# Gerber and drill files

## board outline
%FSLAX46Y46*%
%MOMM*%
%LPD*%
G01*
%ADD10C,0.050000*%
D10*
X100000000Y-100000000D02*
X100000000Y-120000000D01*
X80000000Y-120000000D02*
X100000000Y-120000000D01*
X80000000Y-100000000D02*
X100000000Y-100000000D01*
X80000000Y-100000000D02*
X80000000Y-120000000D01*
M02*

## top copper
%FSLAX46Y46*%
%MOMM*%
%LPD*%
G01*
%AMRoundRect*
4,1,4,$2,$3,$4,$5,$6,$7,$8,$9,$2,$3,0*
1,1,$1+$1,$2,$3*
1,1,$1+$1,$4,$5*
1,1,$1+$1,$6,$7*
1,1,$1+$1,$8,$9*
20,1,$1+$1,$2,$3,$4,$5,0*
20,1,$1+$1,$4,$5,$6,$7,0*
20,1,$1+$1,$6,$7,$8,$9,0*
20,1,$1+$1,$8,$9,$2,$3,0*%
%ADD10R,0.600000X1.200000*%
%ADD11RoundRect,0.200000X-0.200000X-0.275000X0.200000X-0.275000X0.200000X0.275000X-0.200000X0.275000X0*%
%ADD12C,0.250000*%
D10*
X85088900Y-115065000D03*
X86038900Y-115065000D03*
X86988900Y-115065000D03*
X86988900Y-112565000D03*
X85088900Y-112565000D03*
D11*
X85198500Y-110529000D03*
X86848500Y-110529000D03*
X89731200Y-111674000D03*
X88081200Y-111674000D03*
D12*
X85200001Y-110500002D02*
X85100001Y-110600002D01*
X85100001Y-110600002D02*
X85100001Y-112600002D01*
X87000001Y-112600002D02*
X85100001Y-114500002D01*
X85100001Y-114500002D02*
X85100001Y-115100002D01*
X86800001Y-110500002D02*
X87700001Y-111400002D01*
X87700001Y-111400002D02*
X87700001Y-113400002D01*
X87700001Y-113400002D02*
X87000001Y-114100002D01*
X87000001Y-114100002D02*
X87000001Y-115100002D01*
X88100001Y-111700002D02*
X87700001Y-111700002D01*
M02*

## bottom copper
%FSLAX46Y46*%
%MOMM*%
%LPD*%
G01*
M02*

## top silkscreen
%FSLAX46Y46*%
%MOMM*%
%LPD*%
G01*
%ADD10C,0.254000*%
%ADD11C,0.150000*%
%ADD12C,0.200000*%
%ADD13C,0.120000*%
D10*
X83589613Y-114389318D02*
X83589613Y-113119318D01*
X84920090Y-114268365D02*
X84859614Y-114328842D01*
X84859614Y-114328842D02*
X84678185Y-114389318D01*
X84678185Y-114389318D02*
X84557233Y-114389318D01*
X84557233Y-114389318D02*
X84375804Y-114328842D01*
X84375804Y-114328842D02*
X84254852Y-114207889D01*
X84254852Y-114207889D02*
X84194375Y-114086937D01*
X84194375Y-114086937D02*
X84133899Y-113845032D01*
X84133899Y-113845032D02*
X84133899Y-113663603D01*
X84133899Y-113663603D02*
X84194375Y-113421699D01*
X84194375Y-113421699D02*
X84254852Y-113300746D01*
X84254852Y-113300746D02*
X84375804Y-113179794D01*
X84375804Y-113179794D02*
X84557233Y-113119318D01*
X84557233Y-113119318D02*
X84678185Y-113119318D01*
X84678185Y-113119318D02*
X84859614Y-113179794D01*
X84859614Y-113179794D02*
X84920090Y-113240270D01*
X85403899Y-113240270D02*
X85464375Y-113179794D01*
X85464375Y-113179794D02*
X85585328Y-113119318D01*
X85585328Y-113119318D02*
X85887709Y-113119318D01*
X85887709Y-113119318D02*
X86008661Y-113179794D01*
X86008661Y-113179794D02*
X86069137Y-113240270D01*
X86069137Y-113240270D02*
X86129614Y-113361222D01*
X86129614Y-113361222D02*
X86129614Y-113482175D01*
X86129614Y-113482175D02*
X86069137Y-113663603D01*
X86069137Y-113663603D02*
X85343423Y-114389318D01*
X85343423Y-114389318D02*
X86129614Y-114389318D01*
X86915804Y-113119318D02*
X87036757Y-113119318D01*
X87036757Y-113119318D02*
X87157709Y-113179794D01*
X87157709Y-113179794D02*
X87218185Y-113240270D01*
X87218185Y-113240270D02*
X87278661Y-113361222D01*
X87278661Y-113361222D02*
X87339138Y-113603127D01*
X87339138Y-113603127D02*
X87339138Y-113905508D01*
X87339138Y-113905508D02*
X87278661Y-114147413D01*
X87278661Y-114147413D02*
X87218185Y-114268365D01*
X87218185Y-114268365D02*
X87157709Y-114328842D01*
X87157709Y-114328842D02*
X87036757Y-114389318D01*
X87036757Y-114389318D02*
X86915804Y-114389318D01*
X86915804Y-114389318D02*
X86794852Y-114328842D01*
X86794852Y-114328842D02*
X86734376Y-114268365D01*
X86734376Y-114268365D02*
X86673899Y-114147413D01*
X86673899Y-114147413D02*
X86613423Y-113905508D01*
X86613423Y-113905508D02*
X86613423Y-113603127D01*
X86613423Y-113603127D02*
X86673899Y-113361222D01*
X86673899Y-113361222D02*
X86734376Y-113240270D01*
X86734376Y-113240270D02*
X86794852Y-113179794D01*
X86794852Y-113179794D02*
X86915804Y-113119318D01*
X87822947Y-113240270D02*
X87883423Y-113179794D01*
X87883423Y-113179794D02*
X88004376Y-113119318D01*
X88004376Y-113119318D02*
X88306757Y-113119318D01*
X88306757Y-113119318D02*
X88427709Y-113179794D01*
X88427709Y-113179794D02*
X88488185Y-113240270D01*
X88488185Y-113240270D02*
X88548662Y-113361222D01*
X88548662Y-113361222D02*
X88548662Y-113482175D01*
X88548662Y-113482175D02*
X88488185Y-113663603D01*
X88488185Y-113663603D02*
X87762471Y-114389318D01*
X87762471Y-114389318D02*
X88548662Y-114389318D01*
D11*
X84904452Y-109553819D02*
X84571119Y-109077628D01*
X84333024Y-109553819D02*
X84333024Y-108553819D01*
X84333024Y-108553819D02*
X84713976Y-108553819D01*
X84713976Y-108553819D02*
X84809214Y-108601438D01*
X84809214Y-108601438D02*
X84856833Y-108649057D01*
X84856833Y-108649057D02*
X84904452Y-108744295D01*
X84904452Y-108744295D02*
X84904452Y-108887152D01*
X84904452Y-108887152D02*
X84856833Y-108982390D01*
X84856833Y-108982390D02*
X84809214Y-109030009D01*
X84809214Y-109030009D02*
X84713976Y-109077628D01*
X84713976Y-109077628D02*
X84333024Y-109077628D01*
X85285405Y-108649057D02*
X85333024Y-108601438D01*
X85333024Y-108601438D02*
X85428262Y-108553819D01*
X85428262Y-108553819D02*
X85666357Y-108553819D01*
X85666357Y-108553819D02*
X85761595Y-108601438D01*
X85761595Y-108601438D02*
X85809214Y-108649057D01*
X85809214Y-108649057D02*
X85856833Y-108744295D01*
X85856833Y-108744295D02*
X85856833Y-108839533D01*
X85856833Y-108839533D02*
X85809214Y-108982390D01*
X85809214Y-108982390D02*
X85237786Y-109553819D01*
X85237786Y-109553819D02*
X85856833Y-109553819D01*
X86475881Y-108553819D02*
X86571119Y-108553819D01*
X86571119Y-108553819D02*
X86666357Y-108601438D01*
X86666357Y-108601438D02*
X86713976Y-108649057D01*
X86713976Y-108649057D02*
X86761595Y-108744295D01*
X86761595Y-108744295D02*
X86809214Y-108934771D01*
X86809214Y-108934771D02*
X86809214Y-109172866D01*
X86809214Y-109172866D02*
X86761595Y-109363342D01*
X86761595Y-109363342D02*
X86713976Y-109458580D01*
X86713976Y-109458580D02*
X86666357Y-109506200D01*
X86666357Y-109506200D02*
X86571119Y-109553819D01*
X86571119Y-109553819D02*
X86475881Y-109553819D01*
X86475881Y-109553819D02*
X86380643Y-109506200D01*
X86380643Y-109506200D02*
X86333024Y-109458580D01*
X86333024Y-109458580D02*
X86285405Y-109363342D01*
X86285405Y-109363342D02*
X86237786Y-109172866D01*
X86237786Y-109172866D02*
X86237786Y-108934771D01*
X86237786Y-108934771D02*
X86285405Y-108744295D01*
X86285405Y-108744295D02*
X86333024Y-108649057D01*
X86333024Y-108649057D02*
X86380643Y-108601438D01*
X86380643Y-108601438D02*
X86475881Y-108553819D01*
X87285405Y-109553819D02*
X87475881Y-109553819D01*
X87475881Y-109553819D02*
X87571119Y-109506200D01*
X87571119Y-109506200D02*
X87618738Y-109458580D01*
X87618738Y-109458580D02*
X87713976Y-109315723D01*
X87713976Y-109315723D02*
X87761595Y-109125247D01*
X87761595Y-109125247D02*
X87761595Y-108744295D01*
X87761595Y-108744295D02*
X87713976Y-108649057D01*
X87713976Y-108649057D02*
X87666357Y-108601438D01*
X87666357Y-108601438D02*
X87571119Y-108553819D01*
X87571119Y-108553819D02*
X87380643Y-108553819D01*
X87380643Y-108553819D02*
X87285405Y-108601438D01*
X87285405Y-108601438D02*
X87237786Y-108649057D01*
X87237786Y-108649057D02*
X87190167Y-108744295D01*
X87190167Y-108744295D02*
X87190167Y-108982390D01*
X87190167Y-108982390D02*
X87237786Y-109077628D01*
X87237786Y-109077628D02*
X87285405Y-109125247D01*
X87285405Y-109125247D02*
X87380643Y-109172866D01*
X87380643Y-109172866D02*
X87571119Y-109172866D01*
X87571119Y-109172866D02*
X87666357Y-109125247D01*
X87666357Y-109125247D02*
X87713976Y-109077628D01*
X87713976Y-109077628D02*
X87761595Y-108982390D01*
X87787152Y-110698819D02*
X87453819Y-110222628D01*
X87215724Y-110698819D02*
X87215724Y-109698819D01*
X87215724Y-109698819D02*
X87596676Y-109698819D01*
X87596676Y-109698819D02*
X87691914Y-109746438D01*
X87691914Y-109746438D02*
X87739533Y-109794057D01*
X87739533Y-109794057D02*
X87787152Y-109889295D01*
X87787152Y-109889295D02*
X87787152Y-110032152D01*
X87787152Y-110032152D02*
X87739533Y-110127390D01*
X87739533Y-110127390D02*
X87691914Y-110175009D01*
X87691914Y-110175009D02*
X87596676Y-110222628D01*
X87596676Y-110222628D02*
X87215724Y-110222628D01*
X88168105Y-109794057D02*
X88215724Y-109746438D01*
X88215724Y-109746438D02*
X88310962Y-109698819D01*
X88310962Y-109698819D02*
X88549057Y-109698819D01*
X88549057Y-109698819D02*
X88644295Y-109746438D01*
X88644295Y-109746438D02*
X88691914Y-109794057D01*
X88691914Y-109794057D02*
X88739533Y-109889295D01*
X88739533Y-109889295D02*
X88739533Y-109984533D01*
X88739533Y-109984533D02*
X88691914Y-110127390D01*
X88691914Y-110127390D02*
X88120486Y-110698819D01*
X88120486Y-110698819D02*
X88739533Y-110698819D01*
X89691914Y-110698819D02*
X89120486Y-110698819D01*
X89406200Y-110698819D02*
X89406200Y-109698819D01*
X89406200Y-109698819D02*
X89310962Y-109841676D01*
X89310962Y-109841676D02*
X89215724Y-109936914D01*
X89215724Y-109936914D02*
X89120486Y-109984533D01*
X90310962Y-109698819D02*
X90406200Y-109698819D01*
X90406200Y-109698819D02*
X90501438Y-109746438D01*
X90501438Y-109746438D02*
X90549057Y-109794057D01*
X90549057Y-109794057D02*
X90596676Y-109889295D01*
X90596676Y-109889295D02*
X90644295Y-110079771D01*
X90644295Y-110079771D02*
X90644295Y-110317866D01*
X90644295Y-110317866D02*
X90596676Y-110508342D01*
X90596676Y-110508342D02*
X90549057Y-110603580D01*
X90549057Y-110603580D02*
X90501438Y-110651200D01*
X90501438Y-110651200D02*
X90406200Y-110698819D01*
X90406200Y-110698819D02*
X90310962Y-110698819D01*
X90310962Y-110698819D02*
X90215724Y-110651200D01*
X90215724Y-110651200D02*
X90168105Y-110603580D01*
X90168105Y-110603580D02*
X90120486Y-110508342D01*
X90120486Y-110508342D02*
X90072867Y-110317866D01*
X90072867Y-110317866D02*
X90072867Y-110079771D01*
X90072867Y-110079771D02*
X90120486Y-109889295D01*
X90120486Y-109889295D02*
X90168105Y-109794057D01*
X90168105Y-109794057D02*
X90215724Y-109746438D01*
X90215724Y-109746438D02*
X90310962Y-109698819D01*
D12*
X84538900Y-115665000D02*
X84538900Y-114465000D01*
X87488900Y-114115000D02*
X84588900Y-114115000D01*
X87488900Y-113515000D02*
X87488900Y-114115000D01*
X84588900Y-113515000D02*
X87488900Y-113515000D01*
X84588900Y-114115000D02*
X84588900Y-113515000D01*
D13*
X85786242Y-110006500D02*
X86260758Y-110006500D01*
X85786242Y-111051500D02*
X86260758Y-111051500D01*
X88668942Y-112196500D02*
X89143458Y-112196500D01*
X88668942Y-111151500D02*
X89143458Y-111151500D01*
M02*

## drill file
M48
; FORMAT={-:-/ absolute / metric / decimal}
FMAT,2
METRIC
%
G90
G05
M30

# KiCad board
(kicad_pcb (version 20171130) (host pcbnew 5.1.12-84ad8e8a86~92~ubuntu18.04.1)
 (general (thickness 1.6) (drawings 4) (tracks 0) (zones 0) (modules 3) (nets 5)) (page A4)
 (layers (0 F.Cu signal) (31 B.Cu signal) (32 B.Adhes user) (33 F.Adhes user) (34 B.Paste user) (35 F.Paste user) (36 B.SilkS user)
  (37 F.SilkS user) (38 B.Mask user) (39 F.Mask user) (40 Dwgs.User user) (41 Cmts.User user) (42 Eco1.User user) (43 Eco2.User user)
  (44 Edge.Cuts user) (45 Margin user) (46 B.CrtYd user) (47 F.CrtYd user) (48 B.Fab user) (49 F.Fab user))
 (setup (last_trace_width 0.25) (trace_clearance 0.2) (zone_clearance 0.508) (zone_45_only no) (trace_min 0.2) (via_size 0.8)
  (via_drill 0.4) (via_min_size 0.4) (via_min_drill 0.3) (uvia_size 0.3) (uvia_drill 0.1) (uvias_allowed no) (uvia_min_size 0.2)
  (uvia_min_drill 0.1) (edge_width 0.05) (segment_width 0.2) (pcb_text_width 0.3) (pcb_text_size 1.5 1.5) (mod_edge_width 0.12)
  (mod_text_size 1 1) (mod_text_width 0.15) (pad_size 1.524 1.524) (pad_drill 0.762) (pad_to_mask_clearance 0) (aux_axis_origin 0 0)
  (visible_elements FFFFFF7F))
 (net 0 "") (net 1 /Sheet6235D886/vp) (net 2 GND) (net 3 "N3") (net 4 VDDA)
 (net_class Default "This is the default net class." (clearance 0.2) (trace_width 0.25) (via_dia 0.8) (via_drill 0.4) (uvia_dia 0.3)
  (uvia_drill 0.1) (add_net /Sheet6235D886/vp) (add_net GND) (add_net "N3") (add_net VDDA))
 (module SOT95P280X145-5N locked (layer F.Cu) (at 86.038900 113.815000 90.000000)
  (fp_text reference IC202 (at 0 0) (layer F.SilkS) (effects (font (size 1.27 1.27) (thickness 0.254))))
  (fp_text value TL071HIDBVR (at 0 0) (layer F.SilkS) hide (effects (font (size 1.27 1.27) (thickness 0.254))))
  (fp_line (start -1.85 -1.5) (end -0.65 -1.5) (layer F.SilkS) (width 0.2))
  (fp_line (start -0.3 1.45) (end -0.3 -1.45) (layer F.SilkS) (width 0.2))
  (fp_line (start 0.3 1.45) (end -0.3 1.45) (layer F.SilkS) (width 0.2))
  (fp_line (start 0.3 -1.45) (end 0.3 1.45) (layer F.SilkS) (width 0.2))
  (fp_line (start -0.3 -1.45) (end 0.3 -1.45) (layer F.SilkS) (width 0.2))
  (pad 1 smd rect (at -1.25 -0.95 180.000000) (size 0.6 1.2) (layers F.Cu F.Mask F.Paste) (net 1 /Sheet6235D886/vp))
  (pad 2 smd rect (at -1.25 0 180.000000) (size 0.6 1.2) (layers F.Cu F.Mask F.Paste) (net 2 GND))
  (pad 3 smd rect (at -1.25 0.95 180.000000) (size 0.6 1.2) (layers F.Cu F.Mask F.Paste) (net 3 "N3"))
  (pad 4 smd rect (at 1.25 0.95 180.000000) (size 0.6 1.2) (layers F.Cu F.Mask F.Paste) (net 1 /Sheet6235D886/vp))
  (pad 5 smd rect (at 1.25 -0.95 180.000000) (size 0.6 1.2) (layers F.Cu F.Mask F.Paste) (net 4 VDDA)))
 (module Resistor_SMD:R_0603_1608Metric (layer F.Cu) (at 86.023500 110.529000)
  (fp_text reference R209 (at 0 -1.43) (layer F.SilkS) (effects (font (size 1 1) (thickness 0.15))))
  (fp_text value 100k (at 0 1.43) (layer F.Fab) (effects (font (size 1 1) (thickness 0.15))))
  (fp_line (start -0.237258 -0.5225) (end 0.237258 -0.5225) (layer F.SilkS) (width 0.12))
  (fp_line (start -0.237258 0.5225) (end 0.237258 0.5225) (layer F.SilkS) (width 0.12))
  (pad 1 smd roundrect (at -0.825 0) (size 0.8 0.95) (layers F.Cu F.Mask F.Paste) (roundrect_rratio 0.25) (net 4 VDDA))
  (pad 2 smd roundrect (at 0.825 0) (size 0.8 0.95) (layers F.Cu F.Mask F.Paste) (roundrect_rratio 0.25) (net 3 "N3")))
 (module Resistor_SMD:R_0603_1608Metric (layer F.Cu) (at 88.906200 111.674000)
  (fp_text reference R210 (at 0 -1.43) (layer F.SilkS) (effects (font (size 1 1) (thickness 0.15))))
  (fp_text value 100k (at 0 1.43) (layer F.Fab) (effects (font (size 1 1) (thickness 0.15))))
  (fp_line (start -0.237258 0.5225) (end 0.237258 0.5225) (layer F.SilkS) (width 0.12))
  (fp_line (start -0.237258 -0.5225) (end 0.237258 -0.5225) (layer F.SilkS) (width 0.12))
  (pad 2 smd roundrect (at 0.825 0) (size 0.8 0.95) (layers F.Cu F.Mask F.Paste) (roundrect_rratio 0.25) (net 2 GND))
  (pad 1 smd roundrect (at -0.825 0) (size 0.8 0.95) (layers F.Cu F.Mask F.Paste) (roundrect_rratio 0.25) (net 3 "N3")))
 (gr_line (start 100 100) (end 100 120) (layer Edge.Cuts) (width 0.05))
 (gr_line (start 80 120) (end 100 120) (layer Edge.Cuts) (width 0.05))
 (gr_line (start 80 100) (end 100 100) (layer Edge.Cuts) (width 0.05))
 (gr_line (start 80 100) (end 80 120) (layer Edge.Cuts) (width 0.05))
 (segment (start 85.200001 110.500002) (end 85.100001 110.600002) (width 0.250000) (layer F.Cu) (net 4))
 (segment (start 85.100001 110.600002) (end 85.100001 112.600002) (width 0.250000) (layer F.Cu) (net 4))
 (segment (start 87.000001 112.600002) (end 85.100001 114.500002) (width 0.250000) (layer F.Cu) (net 1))
 (segment (start 85.100001 114.500002) (end 85.100001 115.100002) (width 0.250000) (layer F.Cu) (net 1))
 (segment (start 86.800001 110.500002) (end 87.700001 111.400002) (width 0.250000) (layer F.Cu) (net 3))
 (segment (start 87.700001 111.400002) (end 87.700001 113.400002) (width 0.250000) (layer F.Cu) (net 3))
 (segment (start 87.700001 113.400002) (end 87.000001 114.100002) (width 0.250000) (layer F.Cu) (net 3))
 (segment (start 87.000001 114.100002) (end 87.000001 115.100002) (width 0.250000) (layer F.Cu) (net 3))
 (segment (start 88.100001 111.700002) (end 87.700001 111.700002) (width 0.250000) (layer F.Cu) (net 3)))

